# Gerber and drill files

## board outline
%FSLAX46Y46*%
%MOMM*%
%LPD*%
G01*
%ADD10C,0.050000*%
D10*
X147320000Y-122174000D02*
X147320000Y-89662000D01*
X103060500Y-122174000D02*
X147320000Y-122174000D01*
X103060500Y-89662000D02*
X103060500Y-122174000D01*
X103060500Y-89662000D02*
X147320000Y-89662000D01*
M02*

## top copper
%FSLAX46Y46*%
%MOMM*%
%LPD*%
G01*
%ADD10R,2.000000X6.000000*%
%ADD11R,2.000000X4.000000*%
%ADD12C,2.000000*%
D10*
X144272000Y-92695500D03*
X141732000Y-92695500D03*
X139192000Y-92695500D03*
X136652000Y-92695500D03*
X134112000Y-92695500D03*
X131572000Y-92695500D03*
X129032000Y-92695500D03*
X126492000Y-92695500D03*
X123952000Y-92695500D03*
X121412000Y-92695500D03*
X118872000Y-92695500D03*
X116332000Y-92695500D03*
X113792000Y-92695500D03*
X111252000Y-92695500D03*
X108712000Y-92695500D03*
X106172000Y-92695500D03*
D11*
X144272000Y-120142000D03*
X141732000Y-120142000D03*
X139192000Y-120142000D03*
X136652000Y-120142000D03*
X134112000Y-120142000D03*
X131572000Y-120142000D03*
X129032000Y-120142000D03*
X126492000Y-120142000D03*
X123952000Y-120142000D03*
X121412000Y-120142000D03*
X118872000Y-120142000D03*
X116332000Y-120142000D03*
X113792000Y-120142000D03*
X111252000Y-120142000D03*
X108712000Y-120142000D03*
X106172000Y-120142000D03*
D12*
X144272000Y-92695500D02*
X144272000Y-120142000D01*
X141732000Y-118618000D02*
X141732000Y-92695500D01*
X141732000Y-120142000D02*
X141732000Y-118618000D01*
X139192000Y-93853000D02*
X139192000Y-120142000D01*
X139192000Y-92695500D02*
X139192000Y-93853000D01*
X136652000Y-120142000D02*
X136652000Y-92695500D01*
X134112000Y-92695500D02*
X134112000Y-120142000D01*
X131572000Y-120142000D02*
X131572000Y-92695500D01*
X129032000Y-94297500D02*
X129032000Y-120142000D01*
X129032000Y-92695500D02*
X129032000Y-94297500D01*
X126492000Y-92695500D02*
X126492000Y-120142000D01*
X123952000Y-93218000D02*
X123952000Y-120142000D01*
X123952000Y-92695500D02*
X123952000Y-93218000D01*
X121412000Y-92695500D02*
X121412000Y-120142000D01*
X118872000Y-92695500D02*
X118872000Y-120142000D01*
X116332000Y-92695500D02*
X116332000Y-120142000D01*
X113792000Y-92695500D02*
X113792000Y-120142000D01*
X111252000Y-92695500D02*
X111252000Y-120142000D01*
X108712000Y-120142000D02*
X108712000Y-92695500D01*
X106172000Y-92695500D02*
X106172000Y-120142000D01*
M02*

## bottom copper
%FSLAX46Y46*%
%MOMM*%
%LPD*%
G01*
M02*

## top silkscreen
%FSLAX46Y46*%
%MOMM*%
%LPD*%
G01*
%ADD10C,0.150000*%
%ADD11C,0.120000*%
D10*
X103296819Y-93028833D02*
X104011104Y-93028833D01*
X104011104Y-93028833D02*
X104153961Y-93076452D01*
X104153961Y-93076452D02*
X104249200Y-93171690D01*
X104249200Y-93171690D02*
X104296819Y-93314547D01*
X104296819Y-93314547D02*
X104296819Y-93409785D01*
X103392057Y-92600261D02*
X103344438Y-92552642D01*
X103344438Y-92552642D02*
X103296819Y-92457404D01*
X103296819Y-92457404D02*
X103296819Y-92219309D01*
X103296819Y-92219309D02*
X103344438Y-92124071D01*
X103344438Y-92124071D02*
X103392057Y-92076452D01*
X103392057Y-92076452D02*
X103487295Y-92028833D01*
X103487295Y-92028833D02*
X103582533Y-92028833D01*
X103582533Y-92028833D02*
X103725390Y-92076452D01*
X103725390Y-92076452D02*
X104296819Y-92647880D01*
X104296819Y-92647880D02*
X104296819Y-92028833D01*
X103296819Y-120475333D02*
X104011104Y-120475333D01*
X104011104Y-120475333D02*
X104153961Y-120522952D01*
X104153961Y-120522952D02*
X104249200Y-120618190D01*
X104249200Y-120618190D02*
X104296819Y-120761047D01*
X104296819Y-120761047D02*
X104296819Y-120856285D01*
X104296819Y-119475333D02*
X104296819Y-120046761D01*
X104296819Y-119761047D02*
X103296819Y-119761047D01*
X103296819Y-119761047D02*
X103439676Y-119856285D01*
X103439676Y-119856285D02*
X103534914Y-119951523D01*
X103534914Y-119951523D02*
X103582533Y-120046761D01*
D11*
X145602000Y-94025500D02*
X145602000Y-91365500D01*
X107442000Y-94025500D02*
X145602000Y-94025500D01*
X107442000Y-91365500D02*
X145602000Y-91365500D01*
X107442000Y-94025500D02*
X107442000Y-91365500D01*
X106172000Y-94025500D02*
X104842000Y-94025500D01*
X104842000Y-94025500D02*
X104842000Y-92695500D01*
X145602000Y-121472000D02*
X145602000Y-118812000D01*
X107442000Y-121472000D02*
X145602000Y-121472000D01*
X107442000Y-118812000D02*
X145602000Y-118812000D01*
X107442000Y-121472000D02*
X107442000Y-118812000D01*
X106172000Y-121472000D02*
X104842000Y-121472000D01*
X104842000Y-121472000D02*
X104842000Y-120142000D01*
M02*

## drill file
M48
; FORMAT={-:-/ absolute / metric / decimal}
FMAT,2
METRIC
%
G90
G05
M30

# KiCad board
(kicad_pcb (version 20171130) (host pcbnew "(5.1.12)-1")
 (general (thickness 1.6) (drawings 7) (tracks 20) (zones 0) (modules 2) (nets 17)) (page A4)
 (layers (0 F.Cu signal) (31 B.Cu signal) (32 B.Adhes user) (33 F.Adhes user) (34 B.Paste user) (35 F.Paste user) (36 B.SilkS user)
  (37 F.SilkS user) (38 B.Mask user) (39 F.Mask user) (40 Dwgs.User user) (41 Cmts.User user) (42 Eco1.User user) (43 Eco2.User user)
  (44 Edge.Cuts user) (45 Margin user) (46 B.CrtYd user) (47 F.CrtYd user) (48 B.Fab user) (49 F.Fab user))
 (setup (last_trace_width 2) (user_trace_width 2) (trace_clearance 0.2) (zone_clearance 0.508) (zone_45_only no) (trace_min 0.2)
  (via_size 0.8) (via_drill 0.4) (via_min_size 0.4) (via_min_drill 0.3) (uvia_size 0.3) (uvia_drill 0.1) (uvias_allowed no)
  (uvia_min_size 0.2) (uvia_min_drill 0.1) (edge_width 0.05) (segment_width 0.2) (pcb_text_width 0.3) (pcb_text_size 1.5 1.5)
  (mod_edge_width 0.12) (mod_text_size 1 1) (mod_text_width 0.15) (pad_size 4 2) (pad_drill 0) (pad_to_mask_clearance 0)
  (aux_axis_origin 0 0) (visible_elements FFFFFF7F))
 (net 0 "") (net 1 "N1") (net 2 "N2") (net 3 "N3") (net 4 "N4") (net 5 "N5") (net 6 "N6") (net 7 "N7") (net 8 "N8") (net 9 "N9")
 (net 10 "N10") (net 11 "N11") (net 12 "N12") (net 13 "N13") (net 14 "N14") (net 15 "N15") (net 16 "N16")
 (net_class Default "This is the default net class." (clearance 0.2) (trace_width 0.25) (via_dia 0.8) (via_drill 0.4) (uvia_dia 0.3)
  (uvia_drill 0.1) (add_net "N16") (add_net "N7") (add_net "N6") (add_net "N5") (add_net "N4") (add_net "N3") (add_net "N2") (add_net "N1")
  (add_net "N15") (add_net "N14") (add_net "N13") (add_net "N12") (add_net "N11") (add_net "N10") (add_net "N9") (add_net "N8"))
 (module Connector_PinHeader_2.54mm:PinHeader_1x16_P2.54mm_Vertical (layer F.Cu) (at 106.172 92.6955 90)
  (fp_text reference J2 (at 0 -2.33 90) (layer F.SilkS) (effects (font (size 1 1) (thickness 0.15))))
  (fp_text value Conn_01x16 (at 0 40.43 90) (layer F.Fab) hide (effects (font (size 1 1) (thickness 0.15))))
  (fp_line (start -1.33 39.43) (end 1.33 39.43) (layer F.SilkS) (width 0.12))
  (fp_line (start -1.33 1.27) (end -1.33 39.43) (layer F.SilkS) (width 0.12))
  (fp_line (start 1.33 1.27) (end 1.33 39.43) (layer F.SilkS) (width 0.12))
  (fp_line (start -1.33 1.27) (end 1.33 1.27) (layer F.SilkS) (width 0.12))
  (fp_line (start -1.33 0) (end -1.33 -1.33) (layer F.SilkS) (width 0.12))
  (fp_line (start -1.33 -1.33) (end 0 -1.33) (layer F.SilkS) (width 0.12))
  (pad 16 smd rect (at 0 38.1 90) (size 6 2) (layers F.Cu F.Paste F.Mask) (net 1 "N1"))
  (pad 15 smd rect (at 0 35.56 90) (size 6 2) (layers F.Cu F.Paste F.Mask) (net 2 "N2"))
  (pad 14 smd rect (at 0 33.02 90) (size 6 2) (layers F.Cu F.Paste F.Mask) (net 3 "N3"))
  (pad 13 smd rect (at 0 30.48 90) (size 6 2) (layers F.Cu F.Paste F.Mask) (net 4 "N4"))
  (pad 12 smd rect (at 0 27.94 90) (size 6 2) (layers F.Cu F.Paste F.Mask) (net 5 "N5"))
  (pad 11 smd rect (at 0 25.4 90) (size 6 2) (layers F.Cu F.Paste F.Mask) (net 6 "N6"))
  (pad 10 smd rect (at 0 22.86 90) (size 6 2) (layers F.Cu F.Paste F.Mask) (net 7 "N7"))
  (pad 9 smd rect (at 0 20.32 90) (size 6 2) (layers F.Cu F.Paste F.Mask) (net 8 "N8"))
  (pad 8 smd rect (at 0 17.78 90) (size 6 2) (layers F.Cu F.Paste F.Mask) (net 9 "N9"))
  (pad 7 smd rect (at 0 15.24 90) (size 6 2) (layers F.Cu F.Paste F.Mask) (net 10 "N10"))
  (pad 6 smd rect (at 0 12.7 90) (size 6 2) (layers F.Cu F.Paste F.Mask) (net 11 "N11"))
  (pad 5 smd rect (at 0 10.16 90) (size 6 2) (layers F.Cu F.Paste F.Mask) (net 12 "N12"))
  (pad 4 smd rect (at 0 7.62 90) (size 6 2) (layers F.Cu F.Paste F.Mask) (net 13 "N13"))
  (pad 3 smd rect (at 0 5.08 90) (size 6 2) (layers F.Cu F.Paste F.Mask) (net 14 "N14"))
  (pad 2 smd rect (at 0 2.54 90) (size 6 2) (layers F.Cu F.Paste F.Mask) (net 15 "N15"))
  (pad 1 smd rect (at 0 0 90) (size 6 2) (layers F.Cu F.Paste F.Mask) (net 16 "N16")))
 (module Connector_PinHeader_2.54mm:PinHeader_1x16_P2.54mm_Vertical (layer F.Cu) (at 106.172 120.142 90)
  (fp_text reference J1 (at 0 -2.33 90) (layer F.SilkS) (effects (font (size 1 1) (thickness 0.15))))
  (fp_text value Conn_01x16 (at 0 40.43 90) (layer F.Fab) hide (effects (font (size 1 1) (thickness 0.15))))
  (fp_line (start -1.33 39.43) (end 1.33 39.43) (layer F.SilkS) (width 0.12))
  (fp_line (start -1.33 1.27) (end -1.33 39.43) (layer F.SilkS) (width 0.12))
  (fp_line (start 1.33 1.27) (end 1.33 39.43) (layer F.SilkS) (width 0.12))
  (fp_line (start -1.33 1.27) (end 1.33 1.27) (layer F.SilkS) (width 0.12))
  (fp_line (start -1.33 0) (end -1.33 -1.33) (layer F.SilkS) (width 0.12))
  (fp_line (start -1.33 -1.33) (end 0 -1.33) (layer F.SilkS) (width 0.12))
  (pad 16 smd rect (at 0 38.1 90) (size 4 2) (layers F.Cu F.Paste F.Mask) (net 1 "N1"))
  (pad 15 smd rect (at 0 35.56 90) (size 4 2) (layers F.Cu F.Paste F.Mask) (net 2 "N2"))
  (pad 14 smd rect (at 0 33.02 90) (size 4 2) (layers F.Cu F.Paste F.Mask) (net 3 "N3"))
  (pad 13 smd rect (at 0 30.48 90) (size 4 2) (layers F.Cu F.Paste F.Mask) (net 4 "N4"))
  (pad 12 smd rect (at 0 27.94 90) (size 4 2) (layers F.Cu F.Paste F.Mask) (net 5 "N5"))
  (pad 11 smd rect (at 0 25.4 90) (size 4 2) (layers F.Cu F.Paste F.Mask) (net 6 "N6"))
  (pad 10 smd rect (at 0 22.86 90) (size 4 2) (layers F.Cu F.Paste F.Mask) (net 7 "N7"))
  (pad 9 smd rect (at 0 20.32 90) (size 4 2) (layers F.Cu F.Paste F.Mask) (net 8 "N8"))
  (pad 8 smd rect (at 0 17.78 90) (size 4 2) (layers F.Cu F.Paste F.Mask) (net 9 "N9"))
  (pad 7 smd rect (at 0 15.24 90) (size 4 2) (layers F.Cu F.Paste F.Mask) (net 10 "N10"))
  (pad 6 smd rect (at 0 12.7 90) (size 4 2) (layers F.Cu F.Paste F.Mask) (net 11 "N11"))
  (pad 5 smd rect (at 0 10.16 90) (size 4 2) (layers F.Cu F.Paste F.Mask) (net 12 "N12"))
  (pad 4 smd rect (at 0 7.62 90) (size 4 2) (layers F.Cu F.Paste F.Mask) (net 13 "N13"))
  (pad 3 smd rect (at 0 5.08 90) (size 4 2) (layers F.Cu F.Paste F.Mask) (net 14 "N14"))
  (pad 2 smd rect (at 0 2.54 90) (size 4 2) (layers F.Cu F.Paste F.Mask) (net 15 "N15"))
  (pad 1 smd rect (at 0 0 90) (size 4 2) (layers F.Cu F.Paste F.Mask) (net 16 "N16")))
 (gr_line (start 147.32 122.174) (end 147.32 89.662) (layer Edge.Cuts) (width 0.05))
 (gr_line (start 103.0605 122.174) (end 147.32 122.174) (layer Edge.Cuts) (width 0.05))
 (gr_line (start 103.0605 89.662) (end 103.0605 122.174) (layer Edge.Cuts) (width 0.05))
 (gr_line (start 103.0605 89.662) (end 147.32 89.662) (layer Edge.Cuts) (width 0.05))
 (segment (start 144.272 92.6955) (end 144.272 120.142) (width 2) (layer F.Cu) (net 1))
 (segment (start 141.732 118.618) (end 141.732 92.6955) (width 2) (layer F.Cu) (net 2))
 (segment (start 141.732 120.142) (end 141.732 118.618) (width 2) (layer F.Cu) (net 2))
 (segment (start 139.192 93.853) (end 139.192 120.142) (width 2) (layer F.Cu) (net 3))
 (segment (start 139.192 92.6955) (end 139.192 93.853) (width 2) (layer F.Cu) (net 3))
 (segment (start 136.652 120.142) (end 136.652 92.6955) (width 2) (layer F.Cu) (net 4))
 (segment (start 134.112 92.6955) (end 134.112 120.142) (width 2) (layer F.Cu) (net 5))
 (segment (start 131.572 120.142) (end 131.572 92.6955) (width 2) (layer F.Cu) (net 6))
 (segment (start 129.032 94.2975) (end 129.032 120.142) (width 2) (layer F.Cu) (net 7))
 (segment (start 129.032 92.6955) (end 129.032 94.2975) (width 2) (layer F.Cu) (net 7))
 (segment (start 126.492 92.6955) (end 126.492 120.142) (width 2) (layer F.Cu) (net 8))
 (segment (start 123.952 93.218) (end 123.952 120.142) (width 2) (layer F.Cu) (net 9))
 (segment (start 123.952 92.6955) (end 123.952 93.218) (width 2) (layer F.Cu) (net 9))
 (segment (start 121.412 92.6955) (end 121.412 120.142) (width 2) (layer F.Cu) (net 10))
 (segment (start 118.872 92.6955) (end 118.872 120.142) (width 2) (layer F.Cu) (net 11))
 (segment (start 116.332 92.6955) (end 116.332 120.142) (width 2) (layer F.Cu) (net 12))
 (segment (start 113.792 92.6955) (end 113.792 120.142) (width 2) (layer F.Cu) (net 13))
 (segment (start 111.252 92.6955) (end 111.252 120.142) (width 2) (layer F.Cu) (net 14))
 (segment (start 108.712 120.142) (end 108.712 92.6955) (width 2) (layer F.Cu) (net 15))
 (segment (start 106.172 92.6955) (end 106.172 120.142) (width 2) (layer F.Cu) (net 16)))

